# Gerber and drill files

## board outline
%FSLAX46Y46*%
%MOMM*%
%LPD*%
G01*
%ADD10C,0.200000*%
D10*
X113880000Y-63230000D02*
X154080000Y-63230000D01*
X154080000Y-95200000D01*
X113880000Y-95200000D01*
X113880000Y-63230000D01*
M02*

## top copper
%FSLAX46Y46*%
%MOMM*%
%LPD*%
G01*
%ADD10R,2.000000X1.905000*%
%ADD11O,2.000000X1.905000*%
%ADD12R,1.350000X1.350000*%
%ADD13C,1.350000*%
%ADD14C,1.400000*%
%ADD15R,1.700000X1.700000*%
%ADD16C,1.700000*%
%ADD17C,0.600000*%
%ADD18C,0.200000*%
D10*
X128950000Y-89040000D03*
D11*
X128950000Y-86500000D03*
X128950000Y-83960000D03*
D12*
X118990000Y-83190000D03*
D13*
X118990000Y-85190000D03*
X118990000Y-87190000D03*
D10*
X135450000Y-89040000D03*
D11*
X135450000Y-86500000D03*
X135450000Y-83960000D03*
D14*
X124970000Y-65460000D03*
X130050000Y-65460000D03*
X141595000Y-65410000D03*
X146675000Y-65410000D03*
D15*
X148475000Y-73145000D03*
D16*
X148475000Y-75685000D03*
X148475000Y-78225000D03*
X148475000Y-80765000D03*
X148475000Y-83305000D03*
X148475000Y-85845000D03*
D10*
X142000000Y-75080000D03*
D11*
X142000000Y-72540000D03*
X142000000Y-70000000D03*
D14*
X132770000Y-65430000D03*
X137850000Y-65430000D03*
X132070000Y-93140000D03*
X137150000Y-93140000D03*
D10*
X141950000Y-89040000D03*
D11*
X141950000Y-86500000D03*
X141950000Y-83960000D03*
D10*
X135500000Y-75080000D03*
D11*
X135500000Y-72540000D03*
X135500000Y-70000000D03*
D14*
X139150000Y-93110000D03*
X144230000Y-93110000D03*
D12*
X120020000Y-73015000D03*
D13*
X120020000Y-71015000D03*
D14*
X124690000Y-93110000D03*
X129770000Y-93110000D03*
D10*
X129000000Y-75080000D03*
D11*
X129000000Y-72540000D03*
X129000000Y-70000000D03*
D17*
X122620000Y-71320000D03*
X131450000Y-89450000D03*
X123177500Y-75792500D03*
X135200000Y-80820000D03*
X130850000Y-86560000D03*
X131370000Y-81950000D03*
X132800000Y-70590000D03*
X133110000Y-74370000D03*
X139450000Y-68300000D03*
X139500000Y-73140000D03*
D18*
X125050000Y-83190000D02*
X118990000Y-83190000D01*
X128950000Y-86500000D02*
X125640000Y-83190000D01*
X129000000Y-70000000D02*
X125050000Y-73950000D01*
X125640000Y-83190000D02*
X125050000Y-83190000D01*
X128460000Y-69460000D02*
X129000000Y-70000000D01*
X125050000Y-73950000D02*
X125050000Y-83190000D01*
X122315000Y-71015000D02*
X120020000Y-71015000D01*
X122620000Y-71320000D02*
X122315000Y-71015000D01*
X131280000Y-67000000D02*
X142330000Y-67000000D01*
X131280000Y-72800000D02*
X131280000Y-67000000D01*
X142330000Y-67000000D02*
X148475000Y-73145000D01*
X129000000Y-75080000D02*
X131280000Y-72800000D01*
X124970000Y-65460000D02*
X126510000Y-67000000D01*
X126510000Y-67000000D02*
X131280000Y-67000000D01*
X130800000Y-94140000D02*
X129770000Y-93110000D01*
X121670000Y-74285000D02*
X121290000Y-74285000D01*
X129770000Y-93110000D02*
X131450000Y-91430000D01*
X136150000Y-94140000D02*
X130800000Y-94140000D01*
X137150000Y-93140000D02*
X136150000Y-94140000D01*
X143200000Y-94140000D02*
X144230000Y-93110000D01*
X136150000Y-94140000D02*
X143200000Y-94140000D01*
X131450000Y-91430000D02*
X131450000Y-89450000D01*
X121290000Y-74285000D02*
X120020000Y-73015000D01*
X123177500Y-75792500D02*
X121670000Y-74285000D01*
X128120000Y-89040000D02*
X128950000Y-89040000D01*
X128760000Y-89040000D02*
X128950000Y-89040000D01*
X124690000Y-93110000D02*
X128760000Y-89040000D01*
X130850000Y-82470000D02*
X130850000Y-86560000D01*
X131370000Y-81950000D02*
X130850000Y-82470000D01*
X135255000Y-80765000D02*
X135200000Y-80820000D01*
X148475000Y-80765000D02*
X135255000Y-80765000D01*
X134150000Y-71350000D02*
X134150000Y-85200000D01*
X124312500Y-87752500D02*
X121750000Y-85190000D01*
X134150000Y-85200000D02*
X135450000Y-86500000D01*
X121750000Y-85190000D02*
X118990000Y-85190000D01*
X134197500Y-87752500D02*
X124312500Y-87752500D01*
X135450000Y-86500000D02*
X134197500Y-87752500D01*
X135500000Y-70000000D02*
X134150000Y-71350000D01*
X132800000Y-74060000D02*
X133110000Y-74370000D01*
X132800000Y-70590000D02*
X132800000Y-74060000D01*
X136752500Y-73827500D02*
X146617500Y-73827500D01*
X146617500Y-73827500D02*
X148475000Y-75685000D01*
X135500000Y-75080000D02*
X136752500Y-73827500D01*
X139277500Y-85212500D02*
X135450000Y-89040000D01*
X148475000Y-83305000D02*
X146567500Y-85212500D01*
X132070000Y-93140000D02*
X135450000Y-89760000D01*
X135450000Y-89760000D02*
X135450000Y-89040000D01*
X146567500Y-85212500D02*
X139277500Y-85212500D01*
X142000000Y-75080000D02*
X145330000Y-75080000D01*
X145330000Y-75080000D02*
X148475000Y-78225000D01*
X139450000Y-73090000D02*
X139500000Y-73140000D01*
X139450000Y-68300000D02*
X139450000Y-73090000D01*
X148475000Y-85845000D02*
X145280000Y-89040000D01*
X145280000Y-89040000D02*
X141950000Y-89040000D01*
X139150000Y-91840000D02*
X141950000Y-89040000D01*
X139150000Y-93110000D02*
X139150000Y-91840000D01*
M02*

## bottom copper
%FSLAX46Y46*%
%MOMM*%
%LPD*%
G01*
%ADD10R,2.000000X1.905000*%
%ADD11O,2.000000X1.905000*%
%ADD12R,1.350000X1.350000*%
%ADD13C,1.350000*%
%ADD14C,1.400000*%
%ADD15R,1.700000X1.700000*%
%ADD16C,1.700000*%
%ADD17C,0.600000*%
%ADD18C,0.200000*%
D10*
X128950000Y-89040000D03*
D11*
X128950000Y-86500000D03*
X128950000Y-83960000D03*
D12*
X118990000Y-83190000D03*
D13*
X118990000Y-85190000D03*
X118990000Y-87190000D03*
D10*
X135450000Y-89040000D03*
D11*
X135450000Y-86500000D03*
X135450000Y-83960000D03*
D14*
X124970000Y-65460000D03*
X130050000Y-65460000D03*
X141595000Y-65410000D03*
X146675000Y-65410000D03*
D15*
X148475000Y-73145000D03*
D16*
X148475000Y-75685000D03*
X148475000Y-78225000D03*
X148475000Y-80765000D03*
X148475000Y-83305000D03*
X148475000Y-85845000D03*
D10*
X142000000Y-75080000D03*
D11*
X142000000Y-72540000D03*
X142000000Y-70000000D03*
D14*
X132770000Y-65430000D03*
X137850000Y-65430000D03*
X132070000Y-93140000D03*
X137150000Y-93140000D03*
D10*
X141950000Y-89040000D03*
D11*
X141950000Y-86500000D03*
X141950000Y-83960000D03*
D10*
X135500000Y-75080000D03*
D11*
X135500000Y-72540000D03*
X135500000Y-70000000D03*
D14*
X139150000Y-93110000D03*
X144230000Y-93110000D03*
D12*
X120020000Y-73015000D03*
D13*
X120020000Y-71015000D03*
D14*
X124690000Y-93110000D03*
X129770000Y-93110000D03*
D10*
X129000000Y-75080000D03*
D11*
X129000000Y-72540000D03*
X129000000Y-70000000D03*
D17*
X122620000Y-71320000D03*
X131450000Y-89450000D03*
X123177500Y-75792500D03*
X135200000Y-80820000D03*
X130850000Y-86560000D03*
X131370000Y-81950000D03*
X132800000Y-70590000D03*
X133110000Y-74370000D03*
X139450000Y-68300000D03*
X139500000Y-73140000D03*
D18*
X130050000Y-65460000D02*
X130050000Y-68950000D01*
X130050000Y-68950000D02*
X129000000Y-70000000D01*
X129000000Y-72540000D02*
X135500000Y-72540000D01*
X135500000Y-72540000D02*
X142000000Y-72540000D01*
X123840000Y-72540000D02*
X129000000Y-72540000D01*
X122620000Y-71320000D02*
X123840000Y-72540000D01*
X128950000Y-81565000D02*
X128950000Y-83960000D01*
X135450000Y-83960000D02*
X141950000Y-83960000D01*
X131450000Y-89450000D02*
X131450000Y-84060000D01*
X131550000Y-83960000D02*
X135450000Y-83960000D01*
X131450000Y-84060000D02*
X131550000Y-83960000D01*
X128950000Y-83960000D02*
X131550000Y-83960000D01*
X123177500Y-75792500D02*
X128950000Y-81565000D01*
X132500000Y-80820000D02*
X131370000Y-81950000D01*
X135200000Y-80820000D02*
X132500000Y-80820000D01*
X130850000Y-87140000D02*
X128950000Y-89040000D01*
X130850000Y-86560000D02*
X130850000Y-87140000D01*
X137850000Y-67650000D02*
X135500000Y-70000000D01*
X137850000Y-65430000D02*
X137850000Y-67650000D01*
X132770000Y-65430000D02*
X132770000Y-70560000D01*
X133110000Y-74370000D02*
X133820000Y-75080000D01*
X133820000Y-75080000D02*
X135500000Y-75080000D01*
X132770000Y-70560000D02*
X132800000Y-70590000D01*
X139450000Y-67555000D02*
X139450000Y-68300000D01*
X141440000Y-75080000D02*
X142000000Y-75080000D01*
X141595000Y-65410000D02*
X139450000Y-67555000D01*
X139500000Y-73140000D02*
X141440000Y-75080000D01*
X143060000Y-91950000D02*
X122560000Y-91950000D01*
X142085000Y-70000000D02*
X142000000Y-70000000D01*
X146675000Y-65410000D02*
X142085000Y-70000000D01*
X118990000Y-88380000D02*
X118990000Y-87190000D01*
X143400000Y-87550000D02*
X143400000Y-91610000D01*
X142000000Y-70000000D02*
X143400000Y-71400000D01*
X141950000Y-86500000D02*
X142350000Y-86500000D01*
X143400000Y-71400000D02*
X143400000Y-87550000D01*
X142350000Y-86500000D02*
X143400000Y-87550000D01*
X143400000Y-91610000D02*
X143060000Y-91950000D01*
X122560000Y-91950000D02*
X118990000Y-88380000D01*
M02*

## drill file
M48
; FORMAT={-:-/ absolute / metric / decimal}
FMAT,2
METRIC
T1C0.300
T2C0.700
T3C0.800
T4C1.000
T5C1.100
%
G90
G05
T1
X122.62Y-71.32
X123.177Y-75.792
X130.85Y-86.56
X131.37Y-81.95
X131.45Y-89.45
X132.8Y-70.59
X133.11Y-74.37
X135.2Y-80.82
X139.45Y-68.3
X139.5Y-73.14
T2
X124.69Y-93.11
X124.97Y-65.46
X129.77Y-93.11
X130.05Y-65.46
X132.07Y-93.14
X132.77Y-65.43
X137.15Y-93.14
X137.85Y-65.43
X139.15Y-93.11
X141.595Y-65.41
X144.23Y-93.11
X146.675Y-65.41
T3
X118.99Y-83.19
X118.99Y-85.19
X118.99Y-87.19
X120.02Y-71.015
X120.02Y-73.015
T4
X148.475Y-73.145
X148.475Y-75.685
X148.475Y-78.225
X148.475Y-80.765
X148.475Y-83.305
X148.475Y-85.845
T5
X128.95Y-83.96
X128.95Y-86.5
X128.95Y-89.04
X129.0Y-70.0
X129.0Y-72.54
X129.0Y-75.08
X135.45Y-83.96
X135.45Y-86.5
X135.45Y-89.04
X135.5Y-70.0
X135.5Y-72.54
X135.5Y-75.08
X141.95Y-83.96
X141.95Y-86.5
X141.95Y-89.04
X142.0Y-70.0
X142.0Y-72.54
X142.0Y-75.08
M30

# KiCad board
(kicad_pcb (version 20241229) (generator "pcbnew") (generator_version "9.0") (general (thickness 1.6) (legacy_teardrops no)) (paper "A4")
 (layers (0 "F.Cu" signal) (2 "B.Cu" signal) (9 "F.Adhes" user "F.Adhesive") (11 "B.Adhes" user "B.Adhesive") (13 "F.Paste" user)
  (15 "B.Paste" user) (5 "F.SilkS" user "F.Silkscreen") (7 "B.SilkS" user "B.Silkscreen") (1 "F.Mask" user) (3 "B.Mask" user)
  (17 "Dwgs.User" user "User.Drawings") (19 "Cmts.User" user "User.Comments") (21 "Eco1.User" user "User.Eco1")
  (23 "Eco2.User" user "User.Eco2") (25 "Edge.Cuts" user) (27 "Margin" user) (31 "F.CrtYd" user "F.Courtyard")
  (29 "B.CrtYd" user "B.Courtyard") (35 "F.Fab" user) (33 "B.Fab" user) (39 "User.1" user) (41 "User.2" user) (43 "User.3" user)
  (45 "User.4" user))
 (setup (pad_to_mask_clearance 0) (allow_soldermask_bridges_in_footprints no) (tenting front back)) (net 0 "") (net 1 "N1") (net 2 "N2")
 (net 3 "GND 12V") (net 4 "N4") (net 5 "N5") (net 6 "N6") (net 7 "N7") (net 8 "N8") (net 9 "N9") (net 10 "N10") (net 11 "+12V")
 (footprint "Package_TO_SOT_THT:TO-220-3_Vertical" (layer "F.Cu") (at 128.95 89.04 90)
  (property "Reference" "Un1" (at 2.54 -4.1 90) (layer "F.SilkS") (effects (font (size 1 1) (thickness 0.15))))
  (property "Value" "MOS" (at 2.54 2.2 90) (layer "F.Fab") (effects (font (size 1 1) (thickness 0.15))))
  (pad "1" thru_hole rect (at 0 0 90) (size 1.905 2) (drill 1.1) (layers "*.Cu" "*.Mask") (remove_unused_layers no) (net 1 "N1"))
  (pad "2" thru_hole oval (at 2.54 0 90) (size 1.905 2) (drill 1.1) (layers "*.Cu" "*.Mask") (remove_unused_layers no) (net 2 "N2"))
  (pad "3" thru_hole oval (at 5.08 0 90) (size 1.905 2) (drill 1.1) (layers "*.Cu" "*.Mask") (remove_unused_layers no) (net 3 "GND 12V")))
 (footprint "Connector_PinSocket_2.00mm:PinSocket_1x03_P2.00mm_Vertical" (layer "F.Cu") (at 118.99 83.19)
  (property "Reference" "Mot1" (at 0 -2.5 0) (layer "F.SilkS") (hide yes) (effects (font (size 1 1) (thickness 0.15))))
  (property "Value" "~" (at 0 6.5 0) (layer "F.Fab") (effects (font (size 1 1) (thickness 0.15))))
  (pad "1" thru_hole rect (at 0 0) (size 1.35 1.35) (drill 0.8) (layers "*.Cu" "*.Mask") (remove_unused_layers no) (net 2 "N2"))
  (pad "2" thru_hole circle (at 0 2) (size 1.35 1.35) (drill 0.8) (layers "*.Cu" "*.Mask") (remove_unused_layers no) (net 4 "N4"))
  (pad "3" thru_hole circle (at 0 4) (size 1.35 1.35) (drill 0.8) (layers "*.Cu" "*.Mask") (remove_unused_layers no) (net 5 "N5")))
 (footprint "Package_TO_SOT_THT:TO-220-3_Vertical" (layer "F.Cu") (at 135.45 89.04 90)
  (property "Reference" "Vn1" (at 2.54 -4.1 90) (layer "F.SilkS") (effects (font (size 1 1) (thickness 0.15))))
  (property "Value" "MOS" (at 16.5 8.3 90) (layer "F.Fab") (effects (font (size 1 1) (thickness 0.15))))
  (pad "1" thru_hole rect (at 0 0 90) (size 1.905 2) (drill 1.1) (layers "*.Cu" "*.Mask") (remove_unused_layers no) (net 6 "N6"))
  (pad "2" thru_hole oval (at 2.54 0 90) (size 1.905 2) (drill 1.1) (layers "*.Cu" "*.Mask") (remove_unused_layers no) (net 4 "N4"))
  (pad "3" thru_hole oval (at 5.08 0 90) (size 1.905 2) (drill 1.1) (layers "*.Cu" "*.Mask") (remove_unused_layers no) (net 3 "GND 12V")))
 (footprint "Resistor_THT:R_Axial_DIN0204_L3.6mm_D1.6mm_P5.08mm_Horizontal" (layer "F.Cu") (at 124.97 65.46)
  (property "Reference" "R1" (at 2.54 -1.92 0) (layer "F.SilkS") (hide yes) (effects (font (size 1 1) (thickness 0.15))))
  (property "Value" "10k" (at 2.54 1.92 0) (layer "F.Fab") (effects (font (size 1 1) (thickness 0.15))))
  (pad "1" thru_hole circle (at 0 0) (size 1.4 1.4) (drill 0.7) (layers "*.Cu" "*.Mask") (remove_unused_layers no) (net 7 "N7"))
  (pad "2" thru_hole circle (at 5.08 0) (size 1.4 1.4) (drill 0.7) (layers "*.Cu" "*.Mask") (remove_unused_layers no) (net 2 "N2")))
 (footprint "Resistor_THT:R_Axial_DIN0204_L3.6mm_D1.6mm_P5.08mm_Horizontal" (layer "F.Cu") (at 141.595 65.41)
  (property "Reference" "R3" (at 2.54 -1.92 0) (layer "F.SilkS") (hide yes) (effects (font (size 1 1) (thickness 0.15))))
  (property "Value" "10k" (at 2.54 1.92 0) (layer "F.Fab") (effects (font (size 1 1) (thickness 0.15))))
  (pad "1" thru_hole circle (at 0 0) (size 1.4 1.4) (drill 0.7) (layers "*.Cu" "*.Mask") (remove_unused_layers no) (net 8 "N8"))
  (pad "2" thru_hole circle (at 5.08 0) (size 1.4 1.4) (drill 0.7) (layers "*.Cu" "*.Mask") (remove_unused_layers no) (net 5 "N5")))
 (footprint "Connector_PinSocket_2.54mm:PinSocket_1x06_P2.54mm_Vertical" (layer "F.Cu") (at 148.475 73.145)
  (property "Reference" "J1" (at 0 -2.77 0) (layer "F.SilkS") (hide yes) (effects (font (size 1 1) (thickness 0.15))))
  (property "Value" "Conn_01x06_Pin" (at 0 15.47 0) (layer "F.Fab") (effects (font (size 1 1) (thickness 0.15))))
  (pad "1" thru_hole rect (at 0 0) (size 1.7 1.7) (drill 1) (layers "*.Cu" "*.Mask") (remove_unused_layers no) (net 7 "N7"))
  (pad "2" thru_hole circle (at 0 2.54) (size 1.7 1.7) (drill 1) (layers "*.Cu" "*.Mask") (remove_unused_layers no) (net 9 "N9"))
  (pad "3" thru_hole circle (at 0 5.08) (size 1.7 1.7) (drill 1) (layers "*.Cu" "*.Mask") (remove_unused_layers no) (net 8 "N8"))
  (pad "4" thru_hole circle (at 0 7.62) (size 1.7 1.7) (drill 1) (layers "*.Cu" "*.Mask") (remove_unused_layers no) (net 1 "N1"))
  (pad "5" thru_hole circle (at 0 10.16) (size 1.7 1.7) (drill 1) (layers "*.Cu" "*.Mask") (remove_unused_layers no) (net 6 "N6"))
  (pad "6" thru_hole circle (at 0 12.7) (size 1.7 1.7) (drill 1) (layers "*.Cu" "*.Mask") (remove_unused_layers no) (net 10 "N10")))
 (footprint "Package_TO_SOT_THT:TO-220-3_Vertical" (layer "F.Cu") (at 142 75.08 90)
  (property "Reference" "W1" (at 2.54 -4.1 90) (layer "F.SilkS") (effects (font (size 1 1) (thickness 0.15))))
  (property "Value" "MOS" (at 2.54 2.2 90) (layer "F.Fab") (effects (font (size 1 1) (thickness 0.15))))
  (pad "1" thru_hole rect (at 0 0 90) (size 1.905 2) (drill 1.1) (layers "*.Cu" "*.Mask") (remove_unused_layers no) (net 8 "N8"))
  (pad "2" thru_hole oval (at 2.54 0 90) (size 1.905 2) (drill 1.1) (layers "*.Cu" "*.Mask") (remove_unused_layers no) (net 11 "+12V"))
  (pad "3" thru_hole oval (at 5.08 0 90) (size 1.905 2) (drill 1.1) (layers "*.Cu" "*.Mask") (remove_unused_layers no) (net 5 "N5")))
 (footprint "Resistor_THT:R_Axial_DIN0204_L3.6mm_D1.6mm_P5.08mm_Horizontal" (layer "F.Cu") (at 132.77 65.43)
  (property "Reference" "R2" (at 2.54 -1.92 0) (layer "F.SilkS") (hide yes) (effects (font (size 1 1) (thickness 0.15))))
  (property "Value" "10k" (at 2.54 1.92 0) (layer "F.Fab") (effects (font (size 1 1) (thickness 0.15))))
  (pad "1" thru_hole circle (at 0 0) (size 1.4 1.4) (drill 0.7) (layers "*.Cu" "*.Mask") (remove_unused_layers no) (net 9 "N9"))
  (pad "2" thru_hole circle (at 5.08 0) (size 1.4 1.4) (drill 0.7) (layers "*.Cu" "*.Mask") (remove_unused_layers no) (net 4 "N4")))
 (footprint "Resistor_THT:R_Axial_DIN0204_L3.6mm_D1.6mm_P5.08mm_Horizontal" (layer "F.Cu") (at 132.07 93.14)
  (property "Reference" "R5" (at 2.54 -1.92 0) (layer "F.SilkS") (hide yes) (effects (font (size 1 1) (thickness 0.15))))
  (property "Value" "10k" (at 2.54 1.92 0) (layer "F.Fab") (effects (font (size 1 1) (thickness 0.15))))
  (pad "1" thru_hole circle (at 0 0) (size 1.4 1.4) (drill 0.7) (layers "*.Cu" "*.Mask") (remove_unused_layers no) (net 6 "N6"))
  (pad "2" thru_hole circle (at 5.08 0) (size 1.4 1.4) (drill 0.7) (layers "*.Cu" "*.Mask") (remove_unused_layers no) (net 3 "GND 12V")))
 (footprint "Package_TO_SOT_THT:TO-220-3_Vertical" (layer "F.Cu") (at 141.95 89.04 90)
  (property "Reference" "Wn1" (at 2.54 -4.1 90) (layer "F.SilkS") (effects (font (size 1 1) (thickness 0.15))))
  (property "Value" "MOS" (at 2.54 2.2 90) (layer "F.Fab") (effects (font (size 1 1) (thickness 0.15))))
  (pad "1" thru_hole rect (at 0 0 90) (size 1.905 2) (drill 1.1) (layers "*.Cu" "*.Mask") (remove_unused_layers no) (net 10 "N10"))
  (pad "2" thru_hole oval (at 2.54 0 90) (size 1.905 2) (drill 1.1) (layers "*.Cu" "*.Mask") (remove_unused_layers no) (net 5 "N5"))
  (pad "3" thru_hole oval (at 5.08 0 90) (size 1.905 2) (drill 1.1) (layers "*.Cu" "*.Mask") (remove_unused_layers no) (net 3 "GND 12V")))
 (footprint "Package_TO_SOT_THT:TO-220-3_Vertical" (layer "F.Cu") (at 135.5 75.08 90)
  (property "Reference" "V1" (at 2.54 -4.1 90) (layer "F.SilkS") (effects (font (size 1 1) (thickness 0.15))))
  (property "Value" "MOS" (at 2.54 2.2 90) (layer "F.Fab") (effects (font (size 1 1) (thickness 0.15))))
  (pad "1" thru_hole rect (at 0 0 90) (size 1.905 2) (drill 1.1) (layers "*.Cu" "*.Mask") (remove_unused_layers no) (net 9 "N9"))
  (pad "2" thru_hole oval (at 2.54 0 90) (size 1.905 2) (drill 1.1) (layers "*.Cu" "*.Mask") (remove_unused_layers no) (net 11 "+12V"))
  (pad "3" thru_hole oval (at 5.08 0 90) (size 1.905 2) (drill 1.1) (layers "*.Cu" "*.Mask") (remove_unused_layers no) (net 4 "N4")))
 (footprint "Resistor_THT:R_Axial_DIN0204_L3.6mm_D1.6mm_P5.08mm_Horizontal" (layer "F.Cu") (at 139.15 93.11)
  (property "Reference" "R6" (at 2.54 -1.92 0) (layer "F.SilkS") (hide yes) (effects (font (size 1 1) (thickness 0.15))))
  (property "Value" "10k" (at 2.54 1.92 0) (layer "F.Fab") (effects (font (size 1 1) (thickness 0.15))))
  (pad "1" thru_hole circle (at 0 0) (size 1.4 1.4) (drill 0.7) (layers "*.Cu" "*.Mask") (remove_unused_layers no) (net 10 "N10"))
  (pad "2" thru_hole circle (at 5.08 0) (size 1.4 1.4) (drill 0.7) (layers "*.Cu" "*.Mask") (remove_unused_layers no) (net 3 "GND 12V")))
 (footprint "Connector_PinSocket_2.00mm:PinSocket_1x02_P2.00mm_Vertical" (layer "F.Cu") (at 120.02 73.015 180)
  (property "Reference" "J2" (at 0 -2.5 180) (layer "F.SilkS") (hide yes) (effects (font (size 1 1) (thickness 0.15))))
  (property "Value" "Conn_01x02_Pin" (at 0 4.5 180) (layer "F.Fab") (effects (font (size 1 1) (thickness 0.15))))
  (pad "1" thru_hole rect (at 0 0 180) (size 1.35 1.35) (drill 0.8) (layers "*.Cu" "*.Mask") (remove_unused_layers no) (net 3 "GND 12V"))
  (pad "2" thru_hole circle (at 0 2 180) (size 1.35 1.35) (drill 0.8) (layers "*.Cu" "*.Mask") (remove_unused_layers no) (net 11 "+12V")))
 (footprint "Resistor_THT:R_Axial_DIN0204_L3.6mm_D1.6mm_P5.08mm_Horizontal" (layer "F.Cu") (at 124.69 93.11)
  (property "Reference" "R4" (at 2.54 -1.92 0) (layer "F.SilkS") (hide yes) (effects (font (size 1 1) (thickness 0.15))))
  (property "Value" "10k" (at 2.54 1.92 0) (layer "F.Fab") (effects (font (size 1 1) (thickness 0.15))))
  (pad "1" thru_hole circle (at 0 0) (size 1.4 1.4) (drill 0.7) (layers "*.Cu" "*.Mask") (remove_unused_layers no) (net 1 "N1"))
  (pad "2" thru_hole circle (at 5.08 0) (size 1.4 1.4) (drill 0.7) (layers "*.Cu" "*.Mask") (remove_unused_layers no) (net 3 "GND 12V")))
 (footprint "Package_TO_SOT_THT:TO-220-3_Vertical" (layer "F.Cu") (at 129 75.08 90)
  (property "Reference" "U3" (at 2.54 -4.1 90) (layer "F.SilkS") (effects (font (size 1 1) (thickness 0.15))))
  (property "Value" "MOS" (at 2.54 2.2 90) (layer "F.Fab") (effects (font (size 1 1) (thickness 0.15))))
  (pad "1" thru_hole rect (at 0 0 90) (size 1.905 2) (drill 1.1) (layers "*.Cu" "*.Mask") (remove_unused_layers no) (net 7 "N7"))
  (pad "2" thru_hole oval (at 2.54 0 90) (size 1.905 2) (drill 1.1) (layers "*.Cu" "*.Mask") (remove_unused_layers no) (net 11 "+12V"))
  (pad "3" thru_hole oval (at 5.08 0 90) (size 1.905 2) (drill 1.1) (layers "*.Cu" "*.Mask") (remove_unused_layers no) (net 2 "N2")))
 (gr_rect (start 113.88 63.23) (end 154.08 95.2) (stroke (width 0.2) (type solid)) (fill no) (layer "Edge.Cuts"))
 (segment (start 125.05 83.19) (end 118.99 83.19) (width 0.2) (layer "F.Cu") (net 2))
 (segment (start 128.95 86.5) (end 125.64 83.19) (width 0.2) (layer "F.Cu") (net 2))
 (segment (start 129 70) (end 125.05 73.95) (width 0.2) (layer "F.Cu") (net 2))
 (segment (start 125.64 83.19) (end 125.05 83.19) (width 0.2) (layer "F.Cu") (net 2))
 (segment (start 128.46 69.46) (end 129 70) (width 0.2) (layer "F.Cu") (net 2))
 (segment (start 125.05 73.95) (end 125.05 83.19) (width 0.2) (layer "F.Cu") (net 2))
 (segment (start 130.05 65.46) (end 130.05 68.95) (width 0.2) (layer "B.Cu") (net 2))
 (segment (start 130.05 68.95) (end 129 70) (width 0.2) (layer "B.Cu") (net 2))
 (segment (start 122.315 71.015) (end 120.02 71.015) (width 0.2) (layer "F.Cu") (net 11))
 (segment (start 122.62 71.32) (end 122.315 71.015) (width 0.2) (layer "F.Cu") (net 11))
 (via (at 122.62 71.32) (size 0.6) (drill 0.3) (layers "F.Cu" "B.Cu") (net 11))
 (segment (start 129 72.54) (end 135.5 72.54) (width 0.2) (layer "B.Cu") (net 11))
 (segment (start 135.5 72.54) (end 142 72.54) (width 0.2) (layer "B.Cu") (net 11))
 (segment (start 123.84 72.54) (end 129 72.54) (width 0.2) (layer "B.Cu") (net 11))
 (segment (start 122.62 71.32) (end 123.84 72.54) (width 0.2) (layer "B.Cu") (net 11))
 (segment (start 131.28 67) (end 142.33 67) (width 0.2) (layer "F.Cu") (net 7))
 (segment (start 131.28 72.8) (end 131.28 67) (width 0.2) (layer "F.Cu") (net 7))
 (segment (start 142.33 67) (end 148.475 73.145) (width 0.2) (layer "F.Cu") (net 7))
 (segment (start 129 75.08) (end 131.28 72.8) (width 0.2) (layer "F.Cu") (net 7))
 (segment (start 124.97 65.46) (end 126.51 67) (width 0.2) (layer "F.Cu") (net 7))
 (segment (start 126.51 67) (end 131.28 67) (width 0.2) (layer "F.Cu") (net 7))
 (segment (start 130.8 94.14) (end 129.77 93.11) (width 0.2) (layer "F.Cu") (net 3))
 (segment (start 121.67 74.285) (end 121.29 74.285) (width 0.2) (layer "F.Cu") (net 3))
 (segment (start 129.77 93.11) (end 131.45 91.43) (width 0.2) (layer "F.Cu") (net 3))
 (segment (start 136.15 94.14) (end 130.8 94.14) (width 0.2) (layer "F.Cu") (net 3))
 (segment (start 137.15 93.14) (end 136.15 94.14) (width 0.2) (layer "F.Cu") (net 3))
 (segment (start 143.2 94.14) (end 144.23 93.11) (width 0.2) (layer "F.Cu") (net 3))
 (segment (start 136.15 94.14) (end 143.2 94.14) (width 0.2) (layer "F.Cu") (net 3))
 (segment (start 131.45 91.43) (end 131.45 89.45) (width 0.2) (layer "F.Cu") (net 3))
 (segment (start 121.29 74.285) (end 120.02 73.015) (width 0.2) (layer "F.Cu") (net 3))
 (segment (start 123.1775 75.7925) (end 121.67 74.285) (width 0.2) (layer "F.Cu") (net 3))
 (via (at 131.45 89.45) (size 0.6) (drill 0.3) (layers "F.Cu" "B.Cu") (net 3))
 (via (at 123.1775 75.7925) (size 0.6) (drill 0.3) (layers "F.Cu" "B.Cu") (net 3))
 (segment (start 128.95 81.565) (end 128.95 83.96) (width 0.2) (layer "B.Cu") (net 3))
 (segment (start 135.45 83.96) (end 141.95 83.96) (width 0.2) (layer "B.Cu") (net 3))
 (segment (start 131.45 89.45) (end 131.45 84.06) (width 0.2) (layer "B.Cu") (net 3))
 (segment (start 131.55 83.96) (end 135.45 83.96) (width 0.2) (layer "B.Cu") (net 3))
 (segment (start 131.45 84.06) (end 131.55 83.96) (width 0.2) (layer "B.Cu") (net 3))
 (segment (start 128.95 83.96) (end 131.55 83.96) (width 0.2) (layer "B.Cu") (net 3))
 (segment (start 123.1775 75.7925) (end 128.95 81.565) (width 0.2) (layer "B.Cu") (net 3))
 (segment (start 128.12 89.04) (end 128.95 89.04) (width 0.2) (layer "F.Cu") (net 1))
 (segment (start 128.76 89.04) (end 128.95 89.04) (width 0.2) (layer "F.Cu") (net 1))
 (segment (start 124.69 93.11) (end 128.76 89.04) (width 0.2) (layer "F.Cu") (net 1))
 (segment (start 130.85 82.47) (end 130.85 86.56) (width 0.2) (layer "F.Cu") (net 1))
 (segment (start 131.37 81.95) (end 130.85 82.47) (width 0.2) (layer "F.Cu") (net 1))
 (segment (start 135.255 80.765) (end 135.2 80.82) (width 0.2) (layer "F.Cu") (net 1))
 (segment (start 148.475 80.765) (end 135.255 80.765) (width 0.2) (layer "F.Cu") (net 1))
 (via (at 135.2 80.82) (size 0.6) (drill 0.3) (layers "F.Cu" "B.Cu") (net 1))
 (via (at 130.85 86.56) (size 0.6) (drill 0.3) (layers "F.Cu" "B.Cu") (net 1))
 (via (at 131.37 81.95) (size 0.6) (drill 0.3) (layers "F.Cu" "B.Cu") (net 1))
 (segment (start 132.5 80.82) (end 131.37 81.95) (width 0.2) (layer "B.Cu") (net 1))
 (segment (start 135.2 80.82) (end 132.5 80.82) (width 0.2) (layer "B.Cu") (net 1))
 (segment (start 130.85 87.14) (end 128.95 89.04) (width 0.2) (layer "B.Cu") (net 1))
 (segment (start 130.85 86.56) (end 130.85 87.14) (width 0.2) (layer "B.Cu") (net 1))
 (segment (start 134.15 71.35) (end 134.15 85.2) (width 0.2) (layer "F.Cu") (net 4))
 (segment (start 124.3125 87.7525) (end 121.75 85.19) (width 0.2) (layer "F.Cu") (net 4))
 (segment (start 134.15 85.2) (end 135.45 86.5) (width 0.2) (layer "F.Cu") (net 4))
 (segment (start 121.75 85.19) (end 118.99 85.19) (width 0.2) (layer "F.Cu") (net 4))
 (segment (start 134.1975 87.7525) (end 124.3125 87.7525) (width 0.2) (layer "F.Cu") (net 4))
 (segment (start 135.45 86.5) (end 134.1975 87.7525) (width 0.2) (layer "F.Cu") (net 4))
 (segment (start 135.5 70) (end 134.15 71.35) (width 0.2) (layer "F.Cu") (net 4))
 (segment (start 137.85 67.65) (end 135.5 70) (width 0.2) (layer "B.Cu") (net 4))
 (segment (start 137.85 65.43) (end 137.85 67.65) (width 0.2) (layer "B.Cu") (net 4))
 (segment (start 132.8 74.06) (end 133.11 74.37) (width 0.2) (layer "F.Cu") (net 9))
 (segment (start 132.8 70.59) (end 132.8 74.06) (width 0.2) (layer "F.Cu") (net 9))
 (segment (start 136.7525 73.8275) (end 146.6175 73.8275) (width 0.2) (layer "F.Cu") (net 9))
 (segment (start 146.6175 73.8275) (end 148.475 75.685) (width 0.2) (layer "F.Cu") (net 9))
 (segment (start 135.5 75.08) (end 136.7525 73.8275) (width 0.2) (layer "F.Cu") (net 9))
 (via (at 132.8 70.59) (size 0.6) (drill 0.3) (layers "F.Cu" "B.Cu") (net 9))
 (via (at 133.11 74.37) (size 0.6) (drill 0.3) (layers "F.Cu" "B.Cu") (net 9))
 (segment (start 132.77 65.43) (end 132.77 70.56) (width 0.2) (layer "B.Cu") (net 9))
 (segment (start 133.11 74.37) (end 133.82 75.08) (width 0.2) (layer "B.Cu") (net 9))
 (segment (start 133.82 75.08) (end 135.5 75.08) (width 0.2) (layer "B.Cu") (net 9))
 (segment (start 132.77 70.56) (end 132.8 70.59) (width 0.2) (layer "B.Cu") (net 9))
 (segment (start 139.2775 85.2125) (end 135.45 89.04) (width 0.2) (layer "F.Cu") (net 6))
 (segment (start 148.475 83.305) (end 146.5675 85.2125) (width 0.2) (layer "F.Cu") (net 6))
 (segment (start 132.07 93.14) (end 135.45 89.76) (width 0.2) (layer "F.Cu") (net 6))
 (segment (start 135.45 89.76) (end 135.45 89.04) (width 0.2) (layer "F.Cu") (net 6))
 (segment (start 146.5675 85.2125) (end 139.2775 85.2125) (width 0.2) (layer "F.Cu") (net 6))
 (segment (start 142 75.08) (end 145.33 75.08) (width 0.2) (layer "F.Cu") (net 8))
 (segment (start 145.33 75.08) (end 148.475 78.225) (width 0.2) (layer "F.Cu") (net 8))
 (segment (start 139.45 73.09) (end 139.5 73.14) (width 0.2) (layer "F.Cu") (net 8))
 (segment (start 139.45 68.3) (end 139.45 73.09) (width 0.2) (layer "F.Cu") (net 8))
 (via (at 139.45 68.3) (size 0.6) (drill 0.3) (layers "F.Cu" "B.Cu") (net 8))
 (via (at 139.5 73.14) (size 0.6) (drill 0.3) (layers "F.Cu" "B.Cu") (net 8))
 (segment (start 139.45 67.555) (end 139.45 68.3) (width 0.2) (layer "B.Cu") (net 8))
 (segment (start 141.44 75.08) (end 142 75.08) (width 0.2) (layer "B.Cu") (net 8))
 (segment (start 141.595 65.41) (end 139.45 67.555) (width 0.2) (layer "B.Cu") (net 8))
 (segment (start 139.5 73.14) (end 141.44 75.08) (width 0.2) (layer "B.Cu") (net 8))
 (segment (start 143.06 91.95) (end 122.56 91.95) (width 0.2) (layer "B.Cu") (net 5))
 (segment (start 142.085 70) (end 142 70) (width 0.2) (layer "B.Cu") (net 5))
 (segment (start 146.675 65.41) (end 142.085 70) (width 0.2) (layer "B.Cu") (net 5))
 (segment (start 118.99 88.38) (end 118.99 87.19) (width 0.2) (layer "B.Cu") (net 5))
 (segment (start 143.4 87.55) (end 143.4 91.61) (width 0.2) (layer "B.Cu") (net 5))
 (segment (start 142 70) (end 143.4 71.4) (width 0.2) (layer "B.Cu") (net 5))
 (segment (start 141.95 86.5) (end 142.35 86.5) (width 0.2) (layer "B.Cu") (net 5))
 (segment (start 143.4 71.4) (end 143.4 87.55) (width 0.2) (layer "B.Cu") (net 5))
 (segment (start 142.35 86.5) (end 143.4 87.55) (width 0.2) (layer "B.Cu") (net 5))
 (segment (start 143.4 91.61) (end 143.06 91.95) (width 0.2) (layer "B.Cu") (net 5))
 (segment (start 122.56 91.95) (end 118.99 88.38) (width 0.2) (layer "B.Cu") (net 5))
 (segment (start 148.475 85.845) (end 145.28 89.04) (width 0.2) (layer "F.Cu") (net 10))
 (segment (start 145.28 89.04) (end 141.95 89.04) (width 0.2) (layer "F.Cu") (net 10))
 (segment (start 139.15 91.84) (end 141.95 89.04) (width 0.2) (layer "F.Cu") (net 10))
 (segment (start 139.15 93.11) (end 139.15 91.84) (width 0.2) (layer "F.Cu") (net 10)))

